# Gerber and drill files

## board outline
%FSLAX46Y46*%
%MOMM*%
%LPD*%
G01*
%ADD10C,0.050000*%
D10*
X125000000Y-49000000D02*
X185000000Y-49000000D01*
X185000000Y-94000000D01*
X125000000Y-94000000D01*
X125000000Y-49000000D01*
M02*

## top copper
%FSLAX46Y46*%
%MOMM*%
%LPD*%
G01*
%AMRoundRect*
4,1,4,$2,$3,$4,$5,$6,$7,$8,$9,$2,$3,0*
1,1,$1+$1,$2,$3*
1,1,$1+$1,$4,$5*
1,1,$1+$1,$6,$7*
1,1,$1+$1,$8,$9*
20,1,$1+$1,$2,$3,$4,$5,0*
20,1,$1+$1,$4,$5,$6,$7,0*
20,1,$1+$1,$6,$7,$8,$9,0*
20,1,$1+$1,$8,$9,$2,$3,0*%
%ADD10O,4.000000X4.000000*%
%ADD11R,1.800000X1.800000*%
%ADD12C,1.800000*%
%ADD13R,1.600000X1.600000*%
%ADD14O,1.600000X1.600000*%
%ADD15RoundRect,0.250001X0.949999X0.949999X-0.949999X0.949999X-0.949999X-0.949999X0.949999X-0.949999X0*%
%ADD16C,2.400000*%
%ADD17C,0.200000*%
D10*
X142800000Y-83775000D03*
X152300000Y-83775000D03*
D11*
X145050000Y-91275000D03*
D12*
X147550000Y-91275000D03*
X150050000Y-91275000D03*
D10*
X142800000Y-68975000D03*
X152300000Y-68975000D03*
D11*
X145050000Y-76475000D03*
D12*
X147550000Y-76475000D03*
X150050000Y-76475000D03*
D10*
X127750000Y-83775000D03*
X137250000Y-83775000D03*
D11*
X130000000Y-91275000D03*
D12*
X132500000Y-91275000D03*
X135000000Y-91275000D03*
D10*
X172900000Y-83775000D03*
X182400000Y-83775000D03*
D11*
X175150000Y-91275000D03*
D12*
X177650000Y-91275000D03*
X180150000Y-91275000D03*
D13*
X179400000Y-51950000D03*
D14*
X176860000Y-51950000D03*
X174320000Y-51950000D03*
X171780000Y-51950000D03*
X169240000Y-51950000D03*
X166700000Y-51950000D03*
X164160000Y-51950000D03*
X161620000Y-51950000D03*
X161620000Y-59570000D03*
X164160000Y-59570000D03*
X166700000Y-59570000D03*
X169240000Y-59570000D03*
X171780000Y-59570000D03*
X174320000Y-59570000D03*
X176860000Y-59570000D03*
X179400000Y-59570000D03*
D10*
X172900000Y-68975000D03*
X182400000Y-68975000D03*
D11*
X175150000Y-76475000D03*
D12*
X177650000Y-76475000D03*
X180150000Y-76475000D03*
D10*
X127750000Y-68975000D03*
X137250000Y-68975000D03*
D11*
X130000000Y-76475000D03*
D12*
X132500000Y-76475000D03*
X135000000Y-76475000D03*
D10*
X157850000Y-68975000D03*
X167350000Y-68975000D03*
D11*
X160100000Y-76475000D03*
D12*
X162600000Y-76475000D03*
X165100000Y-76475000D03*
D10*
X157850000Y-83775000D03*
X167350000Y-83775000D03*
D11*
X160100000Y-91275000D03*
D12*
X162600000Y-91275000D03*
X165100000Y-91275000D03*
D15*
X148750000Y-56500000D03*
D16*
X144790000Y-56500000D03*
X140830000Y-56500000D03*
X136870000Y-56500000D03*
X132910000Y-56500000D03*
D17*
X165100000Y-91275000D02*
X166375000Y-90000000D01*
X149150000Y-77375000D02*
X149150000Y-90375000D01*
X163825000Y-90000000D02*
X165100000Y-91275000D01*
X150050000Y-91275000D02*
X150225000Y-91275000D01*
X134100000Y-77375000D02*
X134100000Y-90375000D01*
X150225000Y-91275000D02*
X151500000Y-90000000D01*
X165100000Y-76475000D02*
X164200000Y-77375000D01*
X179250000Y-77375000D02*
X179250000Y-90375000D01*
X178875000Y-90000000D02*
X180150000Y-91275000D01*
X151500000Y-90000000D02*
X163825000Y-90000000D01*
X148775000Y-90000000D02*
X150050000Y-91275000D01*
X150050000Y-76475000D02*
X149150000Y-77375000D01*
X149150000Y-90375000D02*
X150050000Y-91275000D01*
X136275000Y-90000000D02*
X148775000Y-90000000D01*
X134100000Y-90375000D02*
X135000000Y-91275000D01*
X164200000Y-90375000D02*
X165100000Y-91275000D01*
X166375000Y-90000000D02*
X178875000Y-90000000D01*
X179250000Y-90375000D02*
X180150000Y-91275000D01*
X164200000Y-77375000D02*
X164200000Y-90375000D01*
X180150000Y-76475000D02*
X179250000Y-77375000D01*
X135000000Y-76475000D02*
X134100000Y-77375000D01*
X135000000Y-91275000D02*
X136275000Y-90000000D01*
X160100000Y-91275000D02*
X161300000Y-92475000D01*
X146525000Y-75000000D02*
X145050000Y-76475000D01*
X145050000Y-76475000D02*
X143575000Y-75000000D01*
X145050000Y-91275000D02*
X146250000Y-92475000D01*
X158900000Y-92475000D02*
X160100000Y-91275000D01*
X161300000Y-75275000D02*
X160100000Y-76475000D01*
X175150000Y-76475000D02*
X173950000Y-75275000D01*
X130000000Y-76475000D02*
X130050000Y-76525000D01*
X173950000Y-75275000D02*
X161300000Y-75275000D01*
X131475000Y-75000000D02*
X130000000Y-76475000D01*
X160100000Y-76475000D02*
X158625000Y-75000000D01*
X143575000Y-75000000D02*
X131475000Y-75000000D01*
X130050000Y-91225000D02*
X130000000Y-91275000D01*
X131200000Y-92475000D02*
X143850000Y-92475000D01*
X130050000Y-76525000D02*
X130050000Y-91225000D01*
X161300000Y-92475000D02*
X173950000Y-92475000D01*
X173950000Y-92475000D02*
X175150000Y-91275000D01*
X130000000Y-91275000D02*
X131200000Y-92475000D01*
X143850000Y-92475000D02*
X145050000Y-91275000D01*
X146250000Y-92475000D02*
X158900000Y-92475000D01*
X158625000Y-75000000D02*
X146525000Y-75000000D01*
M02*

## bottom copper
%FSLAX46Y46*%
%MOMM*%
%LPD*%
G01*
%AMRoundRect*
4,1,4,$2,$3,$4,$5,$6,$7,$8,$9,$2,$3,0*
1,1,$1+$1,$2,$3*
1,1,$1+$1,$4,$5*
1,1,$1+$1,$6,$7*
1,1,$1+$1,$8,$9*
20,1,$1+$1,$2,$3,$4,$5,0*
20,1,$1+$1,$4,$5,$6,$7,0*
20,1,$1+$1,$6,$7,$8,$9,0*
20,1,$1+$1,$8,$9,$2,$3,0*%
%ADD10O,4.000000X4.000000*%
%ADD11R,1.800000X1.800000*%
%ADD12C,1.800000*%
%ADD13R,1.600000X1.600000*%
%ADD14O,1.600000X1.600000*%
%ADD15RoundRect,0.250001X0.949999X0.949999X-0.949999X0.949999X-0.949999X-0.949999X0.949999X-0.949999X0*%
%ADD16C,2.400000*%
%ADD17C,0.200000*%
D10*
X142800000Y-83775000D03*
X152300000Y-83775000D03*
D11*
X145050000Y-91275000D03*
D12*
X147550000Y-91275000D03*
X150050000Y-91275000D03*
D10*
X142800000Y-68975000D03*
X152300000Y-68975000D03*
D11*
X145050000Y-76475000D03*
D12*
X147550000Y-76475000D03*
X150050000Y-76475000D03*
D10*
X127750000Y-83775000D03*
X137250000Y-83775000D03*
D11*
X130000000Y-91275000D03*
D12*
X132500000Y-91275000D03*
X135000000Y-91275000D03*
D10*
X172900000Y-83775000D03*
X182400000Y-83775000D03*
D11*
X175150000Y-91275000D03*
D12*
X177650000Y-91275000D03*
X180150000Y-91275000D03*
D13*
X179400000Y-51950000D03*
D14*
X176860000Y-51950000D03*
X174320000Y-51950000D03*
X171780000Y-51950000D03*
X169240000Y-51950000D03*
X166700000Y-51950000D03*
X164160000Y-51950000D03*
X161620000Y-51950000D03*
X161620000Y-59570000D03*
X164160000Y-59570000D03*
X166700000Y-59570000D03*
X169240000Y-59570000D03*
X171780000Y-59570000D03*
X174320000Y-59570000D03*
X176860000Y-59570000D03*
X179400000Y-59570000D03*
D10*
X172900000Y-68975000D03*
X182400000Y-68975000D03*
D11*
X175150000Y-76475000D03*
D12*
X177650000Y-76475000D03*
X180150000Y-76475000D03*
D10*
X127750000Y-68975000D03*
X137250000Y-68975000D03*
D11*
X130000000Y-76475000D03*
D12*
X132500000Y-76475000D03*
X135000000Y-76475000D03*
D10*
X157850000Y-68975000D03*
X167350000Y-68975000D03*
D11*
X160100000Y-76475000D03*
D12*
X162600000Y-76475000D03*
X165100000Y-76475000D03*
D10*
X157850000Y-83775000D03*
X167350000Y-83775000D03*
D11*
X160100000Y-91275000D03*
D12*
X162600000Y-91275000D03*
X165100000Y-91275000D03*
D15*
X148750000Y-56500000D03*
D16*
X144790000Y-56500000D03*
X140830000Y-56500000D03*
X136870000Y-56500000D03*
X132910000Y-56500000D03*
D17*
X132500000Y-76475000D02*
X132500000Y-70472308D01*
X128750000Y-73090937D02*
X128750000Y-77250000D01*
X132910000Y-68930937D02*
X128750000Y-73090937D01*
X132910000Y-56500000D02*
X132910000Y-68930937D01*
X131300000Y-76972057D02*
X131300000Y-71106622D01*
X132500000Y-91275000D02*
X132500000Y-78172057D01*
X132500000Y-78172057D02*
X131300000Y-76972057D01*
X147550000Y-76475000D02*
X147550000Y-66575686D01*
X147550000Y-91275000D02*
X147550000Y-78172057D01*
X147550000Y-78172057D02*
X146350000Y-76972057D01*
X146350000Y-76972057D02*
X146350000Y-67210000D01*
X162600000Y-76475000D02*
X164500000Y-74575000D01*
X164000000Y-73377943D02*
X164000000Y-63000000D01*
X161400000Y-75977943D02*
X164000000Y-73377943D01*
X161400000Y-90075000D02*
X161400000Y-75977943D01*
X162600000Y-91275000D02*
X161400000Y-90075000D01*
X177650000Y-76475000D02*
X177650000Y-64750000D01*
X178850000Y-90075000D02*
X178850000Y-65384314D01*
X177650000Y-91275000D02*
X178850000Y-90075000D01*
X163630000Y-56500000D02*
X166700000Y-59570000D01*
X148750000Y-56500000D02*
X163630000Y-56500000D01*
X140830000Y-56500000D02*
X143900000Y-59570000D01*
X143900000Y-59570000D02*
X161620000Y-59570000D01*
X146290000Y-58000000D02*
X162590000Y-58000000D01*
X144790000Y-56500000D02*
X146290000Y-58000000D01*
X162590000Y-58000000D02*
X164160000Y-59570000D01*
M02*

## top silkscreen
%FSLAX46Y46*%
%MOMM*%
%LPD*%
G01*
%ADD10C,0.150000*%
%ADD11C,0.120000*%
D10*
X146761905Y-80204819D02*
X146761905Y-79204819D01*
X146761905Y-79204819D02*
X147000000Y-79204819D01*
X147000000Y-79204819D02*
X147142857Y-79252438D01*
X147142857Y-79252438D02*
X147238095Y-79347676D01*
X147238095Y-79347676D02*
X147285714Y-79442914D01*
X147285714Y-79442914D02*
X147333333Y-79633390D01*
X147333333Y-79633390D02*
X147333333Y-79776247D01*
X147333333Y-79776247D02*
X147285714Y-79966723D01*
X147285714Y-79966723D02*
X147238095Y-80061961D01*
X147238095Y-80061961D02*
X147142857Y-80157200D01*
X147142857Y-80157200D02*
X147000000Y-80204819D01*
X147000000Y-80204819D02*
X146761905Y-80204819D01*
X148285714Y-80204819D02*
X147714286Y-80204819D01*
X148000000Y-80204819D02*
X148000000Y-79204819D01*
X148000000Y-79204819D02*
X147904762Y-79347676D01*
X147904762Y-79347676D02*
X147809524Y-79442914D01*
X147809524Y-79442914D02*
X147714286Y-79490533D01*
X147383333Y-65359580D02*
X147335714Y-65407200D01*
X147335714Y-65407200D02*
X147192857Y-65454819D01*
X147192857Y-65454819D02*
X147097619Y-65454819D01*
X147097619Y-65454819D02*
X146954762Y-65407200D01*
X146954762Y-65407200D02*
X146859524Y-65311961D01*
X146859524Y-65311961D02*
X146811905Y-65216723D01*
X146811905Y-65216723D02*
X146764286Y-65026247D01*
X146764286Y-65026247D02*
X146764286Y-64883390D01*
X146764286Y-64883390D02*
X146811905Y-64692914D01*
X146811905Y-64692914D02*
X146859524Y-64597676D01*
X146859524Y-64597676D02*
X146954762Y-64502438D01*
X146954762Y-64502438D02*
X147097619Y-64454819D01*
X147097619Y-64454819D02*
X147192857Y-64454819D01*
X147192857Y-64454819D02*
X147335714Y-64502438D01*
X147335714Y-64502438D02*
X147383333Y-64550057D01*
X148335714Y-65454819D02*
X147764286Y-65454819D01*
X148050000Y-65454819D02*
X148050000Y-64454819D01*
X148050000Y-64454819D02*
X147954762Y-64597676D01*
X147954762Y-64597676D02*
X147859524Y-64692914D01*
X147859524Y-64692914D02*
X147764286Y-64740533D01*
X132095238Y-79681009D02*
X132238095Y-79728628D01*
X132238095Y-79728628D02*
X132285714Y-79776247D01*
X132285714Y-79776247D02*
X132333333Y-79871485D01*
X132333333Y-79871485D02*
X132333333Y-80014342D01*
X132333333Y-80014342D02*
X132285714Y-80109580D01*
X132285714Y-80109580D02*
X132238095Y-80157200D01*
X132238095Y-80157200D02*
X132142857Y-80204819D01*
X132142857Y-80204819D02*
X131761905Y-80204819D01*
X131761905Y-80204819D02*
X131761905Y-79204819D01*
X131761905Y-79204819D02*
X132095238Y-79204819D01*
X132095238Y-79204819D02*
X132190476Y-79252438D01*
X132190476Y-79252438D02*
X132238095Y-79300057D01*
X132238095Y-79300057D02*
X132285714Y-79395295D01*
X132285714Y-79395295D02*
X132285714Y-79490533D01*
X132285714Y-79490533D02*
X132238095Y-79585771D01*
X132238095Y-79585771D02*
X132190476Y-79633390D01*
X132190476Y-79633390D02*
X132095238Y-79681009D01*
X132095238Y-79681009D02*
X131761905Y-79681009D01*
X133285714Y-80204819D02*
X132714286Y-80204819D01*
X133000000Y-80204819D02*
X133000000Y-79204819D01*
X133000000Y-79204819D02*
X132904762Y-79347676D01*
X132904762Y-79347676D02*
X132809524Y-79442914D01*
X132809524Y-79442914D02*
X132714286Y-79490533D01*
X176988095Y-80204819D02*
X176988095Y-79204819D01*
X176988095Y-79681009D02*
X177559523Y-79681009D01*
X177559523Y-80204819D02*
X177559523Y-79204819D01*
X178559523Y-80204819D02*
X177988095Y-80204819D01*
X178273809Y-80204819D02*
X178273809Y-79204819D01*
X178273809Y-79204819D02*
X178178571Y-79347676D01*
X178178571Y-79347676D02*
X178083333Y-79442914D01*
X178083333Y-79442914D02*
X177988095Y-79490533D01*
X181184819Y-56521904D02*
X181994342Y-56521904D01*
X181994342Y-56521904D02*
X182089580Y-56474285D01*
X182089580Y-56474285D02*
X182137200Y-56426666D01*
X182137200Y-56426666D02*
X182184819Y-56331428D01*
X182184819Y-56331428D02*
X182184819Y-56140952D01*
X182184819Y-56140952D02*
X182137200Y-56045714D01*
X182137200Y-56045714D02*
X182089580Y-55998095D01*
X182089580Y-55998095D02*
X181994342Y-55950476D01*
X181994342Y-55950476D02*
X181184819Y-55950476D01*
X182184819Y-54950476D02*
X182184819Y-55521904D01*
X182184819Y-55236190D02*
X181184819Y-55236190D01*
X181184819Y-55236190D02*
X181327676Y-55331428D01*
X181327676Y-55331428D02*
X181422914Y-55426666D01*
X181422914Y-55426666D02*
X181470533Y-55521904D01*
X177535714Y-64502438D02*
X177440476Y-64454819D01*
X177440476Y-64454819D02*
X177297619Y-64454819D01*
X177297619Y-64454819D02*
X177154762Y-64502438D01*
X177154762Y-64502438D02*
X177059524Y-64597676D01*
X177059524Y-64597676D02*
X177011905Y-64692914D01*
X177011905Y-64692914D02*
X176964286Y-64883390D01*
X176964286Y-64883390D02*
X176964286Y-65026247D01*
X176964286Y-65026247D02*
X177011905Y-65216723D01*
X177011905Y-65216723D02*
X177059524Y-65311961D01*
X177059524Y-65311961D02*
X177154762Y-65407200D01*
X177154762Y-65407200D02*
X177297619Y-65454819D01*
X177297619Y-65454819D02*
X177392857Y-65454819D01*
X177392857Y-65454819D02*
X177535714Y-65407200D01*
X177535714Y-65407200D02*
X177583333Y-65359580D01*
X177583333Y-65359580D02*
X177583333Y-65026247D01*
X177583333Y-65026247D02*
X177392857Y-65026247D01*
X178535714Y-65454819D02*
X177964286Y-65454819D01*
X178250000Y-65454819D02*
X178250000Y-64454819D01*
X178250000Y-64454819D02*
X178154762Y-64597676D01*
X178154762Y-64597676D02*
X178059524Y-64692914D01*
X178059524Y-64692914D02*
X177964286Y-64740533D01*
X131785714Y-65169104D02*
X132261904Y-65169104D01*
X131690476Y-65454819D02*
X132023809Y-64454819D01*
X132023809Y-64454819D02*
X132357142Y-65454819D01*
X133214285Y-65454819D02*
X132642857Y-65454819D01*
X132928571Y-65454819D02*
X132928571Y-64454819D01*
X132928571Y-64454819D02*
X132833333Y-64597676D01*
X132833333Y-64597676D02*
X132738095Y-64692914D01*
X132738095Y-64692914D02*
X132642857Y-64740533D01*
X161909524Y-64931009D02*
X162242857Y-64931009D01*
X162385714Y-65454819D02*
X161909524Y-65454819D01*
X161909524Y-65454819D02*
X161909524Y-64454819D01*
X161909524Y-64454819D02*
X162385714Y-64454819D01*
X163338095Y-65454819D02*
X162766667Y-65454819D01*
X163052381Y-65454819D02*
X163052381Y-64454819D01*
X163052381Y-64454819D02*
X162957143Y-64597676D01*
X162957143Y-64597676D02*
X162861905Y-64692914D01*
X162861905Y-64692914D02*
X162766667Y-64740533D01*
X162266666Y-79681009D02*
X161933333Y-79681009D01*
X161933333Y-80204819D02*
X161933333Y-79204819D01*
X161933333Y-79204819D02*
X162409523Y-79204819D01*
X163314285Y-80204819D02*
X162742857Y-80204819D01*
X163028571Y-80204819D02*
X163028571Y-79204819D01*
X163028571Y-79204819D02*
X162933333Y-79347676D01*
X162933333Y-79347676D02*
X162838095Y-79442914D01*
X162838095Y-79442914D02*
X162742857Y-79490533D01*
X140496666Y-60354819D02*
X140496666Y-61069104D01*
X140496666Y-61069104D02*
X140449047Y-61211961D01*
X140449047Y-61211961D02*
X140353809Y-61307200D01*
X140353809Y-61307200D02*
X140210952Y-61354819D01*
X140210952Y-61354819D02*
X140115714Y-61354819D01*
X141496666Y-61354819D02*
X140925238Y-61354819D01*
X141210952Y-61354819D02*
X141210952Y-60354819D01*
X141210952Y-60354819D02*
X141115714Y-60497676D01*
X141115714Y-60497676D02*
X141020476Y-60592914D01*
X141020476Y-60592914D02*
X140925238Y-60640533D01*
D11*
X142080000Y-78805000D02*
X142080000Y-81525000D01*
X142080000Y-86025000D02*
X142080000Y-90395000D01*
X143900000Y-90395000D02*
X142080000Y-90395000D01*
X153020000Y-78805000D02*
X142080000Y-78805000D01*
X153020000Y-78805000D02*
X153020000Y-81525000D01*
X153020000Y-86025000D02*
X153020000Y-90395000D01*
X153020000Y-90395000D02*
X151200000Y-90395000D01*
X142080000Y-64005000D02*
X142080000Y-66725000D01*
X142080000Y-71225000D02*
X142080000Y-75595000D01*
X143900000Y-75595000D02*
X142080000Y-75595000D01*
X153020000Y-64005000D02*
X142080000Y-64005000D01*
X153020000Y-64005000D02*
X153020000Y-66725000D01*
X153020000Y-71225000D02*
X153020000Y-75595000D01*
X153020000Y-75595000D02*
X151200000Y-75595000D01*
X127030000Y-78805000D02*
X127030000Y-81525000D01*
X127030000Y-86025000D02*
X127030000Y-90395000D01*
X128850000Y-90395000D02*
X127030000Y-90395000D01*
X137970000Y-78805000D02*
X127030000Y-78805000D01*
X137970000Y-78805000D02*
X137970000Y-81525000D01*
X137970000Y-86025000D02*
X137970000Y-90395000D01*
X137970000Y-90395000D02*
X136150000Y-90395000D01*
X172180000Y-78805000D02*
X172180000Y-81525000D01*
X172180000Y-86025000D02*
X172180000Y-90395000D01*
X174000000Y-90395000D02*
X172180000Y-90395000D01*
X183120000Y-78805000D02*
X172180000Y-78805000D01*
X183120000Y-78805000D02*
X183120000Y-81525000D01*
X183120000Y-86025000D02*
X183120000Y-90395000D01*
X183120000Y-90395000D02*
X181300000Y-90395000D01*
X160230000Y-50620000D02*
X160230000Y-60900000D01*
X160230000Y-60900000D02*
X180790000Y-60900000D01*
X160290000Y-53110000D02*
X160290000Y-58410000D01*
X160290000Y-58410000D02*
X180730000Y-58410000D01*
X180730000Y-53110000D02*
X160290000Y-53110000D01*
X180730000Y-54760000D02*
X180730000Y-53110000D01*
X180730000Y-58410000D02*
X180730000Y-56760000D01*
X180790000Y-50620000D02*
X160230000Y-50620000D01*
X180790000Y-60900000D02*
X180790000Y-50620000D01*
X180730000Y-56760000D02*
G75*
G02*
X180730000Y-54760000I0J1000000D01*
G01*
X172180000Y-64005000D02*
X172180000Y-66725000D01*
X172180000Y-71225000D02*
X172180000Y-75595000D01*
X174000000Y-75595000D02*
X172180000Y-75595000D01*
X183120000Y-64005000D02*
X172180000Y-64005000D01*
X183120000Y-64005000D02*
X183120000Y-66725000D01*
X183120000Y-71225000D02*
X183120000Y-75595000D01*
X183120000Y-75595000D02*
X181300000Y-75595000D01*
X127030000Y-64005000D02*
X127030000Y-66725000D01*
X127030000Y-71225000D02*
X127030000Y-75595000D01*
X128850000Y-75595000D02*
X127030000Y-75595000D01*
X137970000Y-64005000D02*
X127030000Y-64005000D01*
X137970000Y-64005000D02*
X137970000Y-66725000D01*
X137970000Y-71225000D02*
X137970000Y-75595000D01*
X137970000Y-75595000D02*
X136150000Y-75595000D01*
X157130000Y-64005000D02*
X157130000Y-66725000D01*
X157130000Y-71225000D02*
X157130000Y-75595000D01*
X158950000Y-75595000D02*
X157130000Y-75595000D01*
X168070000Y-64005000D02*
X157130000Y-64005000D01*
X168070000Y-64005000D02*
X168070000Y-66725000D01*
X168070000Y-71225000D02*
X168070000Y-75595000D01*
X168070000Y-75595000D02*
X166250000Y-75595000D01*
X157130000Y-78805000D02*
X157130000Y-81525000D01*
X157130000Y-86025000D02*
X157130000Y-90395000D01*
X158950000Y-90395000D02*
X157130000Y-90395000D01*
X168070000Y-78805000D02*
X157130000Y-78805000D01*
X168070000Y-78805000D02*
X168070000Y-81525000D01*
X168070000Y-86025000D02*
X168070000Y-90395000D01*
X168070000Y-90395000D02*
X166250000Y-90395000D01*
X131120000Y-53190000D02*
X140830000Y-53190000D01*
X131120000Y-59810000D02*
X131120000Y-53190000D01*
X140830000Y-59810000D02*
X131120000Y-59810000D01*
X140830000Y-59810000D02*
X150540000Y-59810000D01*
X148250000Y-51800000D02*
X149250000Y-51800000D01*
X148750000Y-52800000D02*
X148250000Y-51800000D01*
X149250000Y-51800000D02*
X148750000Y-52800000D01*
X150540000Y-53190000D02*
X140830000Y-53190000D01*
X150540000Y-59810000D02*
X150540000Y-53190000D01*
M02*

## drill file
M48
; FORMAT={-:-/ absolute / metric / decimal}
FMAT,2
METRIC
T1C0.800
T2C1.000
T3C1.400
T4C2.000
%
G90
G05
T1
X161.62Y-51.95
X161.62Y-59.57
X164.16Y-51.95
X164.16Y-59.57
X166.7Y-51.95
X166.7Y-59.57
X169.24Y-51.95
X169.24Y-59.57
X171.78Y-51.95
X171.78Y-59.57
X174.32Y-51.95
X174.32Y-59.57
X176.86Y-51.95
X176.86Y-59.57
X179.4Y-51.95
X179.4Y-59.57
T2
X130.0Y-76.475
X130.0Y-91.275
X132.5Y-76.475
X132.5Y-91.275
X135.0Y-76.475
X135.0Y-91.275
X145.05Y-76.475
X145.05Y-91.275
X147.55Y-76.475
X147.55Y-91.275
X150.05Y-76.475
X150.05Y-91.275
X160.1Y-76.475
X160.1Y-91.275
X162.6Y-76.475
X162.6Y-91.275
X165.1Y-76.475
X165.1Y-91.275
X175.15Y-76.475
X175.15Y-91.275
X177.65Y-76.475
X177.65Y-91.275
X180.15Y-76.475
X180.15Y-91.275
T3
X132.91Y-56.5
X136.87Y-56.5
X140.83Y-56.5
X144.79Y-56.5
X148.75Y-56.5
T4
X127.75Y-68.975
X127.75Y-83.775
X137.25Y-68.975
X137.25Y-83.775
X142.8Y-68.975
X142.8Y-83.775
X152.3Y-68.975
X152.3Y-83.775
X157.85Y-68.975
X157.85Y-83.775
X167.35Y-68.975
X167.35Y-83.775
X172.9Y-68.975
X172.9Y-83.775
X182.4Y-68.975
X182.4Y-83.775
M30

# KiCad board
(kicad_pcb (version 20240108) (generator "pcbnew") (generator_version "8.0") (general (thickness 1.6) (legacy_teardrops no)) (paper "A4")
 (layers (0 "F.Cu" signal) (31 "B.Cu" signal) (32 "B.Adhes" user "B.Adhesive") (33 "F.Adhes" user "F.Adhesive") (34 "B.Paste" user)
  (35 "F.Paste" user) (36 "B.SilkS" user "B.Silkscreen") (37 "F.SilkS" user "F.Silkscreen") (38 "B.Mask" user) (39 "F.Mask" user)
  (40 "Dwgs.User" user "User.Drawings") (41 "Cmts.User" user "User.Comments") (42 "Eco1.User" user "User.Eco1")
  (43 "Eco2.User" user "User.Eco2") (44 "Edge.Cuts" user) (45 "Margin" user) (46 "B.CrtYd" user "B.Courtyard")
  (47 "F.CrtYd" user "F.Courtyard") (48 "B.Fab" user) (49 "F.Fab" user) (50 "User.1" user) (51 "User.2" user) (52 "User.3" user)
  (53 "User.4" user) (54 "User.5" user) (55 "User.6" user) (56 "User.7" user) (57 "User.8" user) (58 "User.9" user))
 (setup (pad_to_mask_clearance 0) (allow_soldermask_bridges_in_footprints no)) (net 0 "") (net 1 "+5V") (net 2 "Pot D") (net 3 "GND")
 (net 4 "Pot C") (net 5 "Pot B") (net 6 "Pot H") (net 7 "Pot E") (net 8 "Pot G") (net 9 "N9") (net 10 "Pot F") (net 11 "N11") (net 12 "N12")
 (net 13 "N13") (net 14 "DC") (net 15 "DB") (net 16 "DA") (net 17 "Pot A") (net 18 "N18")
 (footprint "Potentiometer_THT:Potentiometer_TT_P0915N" (layer "F.Cu") (at 145.05 91.275)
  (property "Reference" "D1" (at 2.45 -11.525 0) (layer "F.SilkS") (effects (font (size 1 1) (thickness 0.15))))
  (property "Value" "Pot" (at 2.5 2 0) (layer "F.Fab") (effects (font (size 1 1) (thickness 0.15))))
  (fp_line (start -2.97 -12.47) (end -2.97 -9.75) (stroke (width 0.12) (type solid)) (layer "F.SilkS"))
  (fp_line (start -2.97 -5.25) (end -2.97 -0.88) (stroke (width 0.12) (type solid)) (layer "F.SilkS"))
  (fp_line (start -1.15 -0.88) (end -2.97 -0.88) (stroke (width 0.12) (type solid)) (layer "F.SilkS"))
  (fp_line (start 7.97 -12.47) (end -2.97 -12.47) (stroke (width 0.12) (type solid)) (layer "F.SilkS"))
  (fp_line (start 7.97 -12.47) (end 7.97 -9.75) (stroke (width 0.12) (type solid)) (layer "F.SilkS"))
  (fp_line (start 7.97 -5.25) (end 7.97 -0.88) (stroke (width 0.12) (type solid)) (layer "F.SilkS"))
  (fp_line (start 7.97 -0.88) (end 6.15 -0.88) (stroke (width 0.12) (type solid)) (layer "F.SilkS"))
  (pad "" thru_hole oval (at -2.25 -7.5) (size 4 4) (drill 2) (layers "*.Cu" "*.Mask") (remove_unused_layers no))
  (pad "" thru_hole oval (at 7.25 -7.5) (size 4 4) (drill 2) (layers "*.Cu" "*.Mask") (remove_unused_layers no))
  (pad "1" thru_hole rect (at 0 0) (size 1.8 1.8) (drill 1) (layers "*.Cu" "*.Mask") (remove_unused_layers no) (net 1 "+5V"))
  (pad "2" thru_hole circle (at 2.5 0) (size 1.8 1.8) (drill 1) (layers "*.Cu" "*.Mask") (remove_unused_layers no) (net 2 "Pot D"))
  (pad "3" thru_hole circle (at 5 0) (size 1.8 1.8) (drill 1) (layers "*.Cu" "*.Mask") (remove_unused_layers no) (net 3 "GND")))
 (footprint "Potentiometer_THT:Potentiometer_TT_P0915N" (layer "F.Cu") (at 145.05 76.475)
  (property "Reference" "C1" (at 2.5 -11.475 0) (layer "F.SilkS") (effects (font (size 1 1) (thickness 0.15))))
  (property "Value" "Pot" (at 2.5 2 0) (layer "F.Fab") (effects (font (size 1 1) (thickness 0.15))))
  (fp_line (start -2.97 -12.47) (end -2.97 -9.75) (stroke (width 0.12) (type solid)) (layer "F.SilkS"))
  (fp_line (start -2.97 -5.25) (end -2.97 -0.88) (stroke (width 0.12) (type solid)) (layer "F.SilkS"))
  (fp_line (start -1.15 -0.88) (end -2.97 -0.88) (stroke (width 0.12) (type solid)) (layer "F.SilkS"))
  (fp_line (start 7.97 -12.47) (end -2.97 -12.47) (stroke (width 0.12) (type solid)) (layer "F.SilkS"))
  (fp_line (start 7.97 -12.47) (end 7.97 -9.75) (stroke (width 0.12) (type solid)) (layer "F.SilkS"))
  (fp_line (start 7.97 -5.25) (end 7.97 -0.88) (stroke (width 0.12) (type solid)) (layer "F.SilkS"))
  (fp_line (start 7.97 -0.88) (end 6.15 -0.88) (stroke (width 0.12) (type solid)) (layer "F.SilkS"))
  (pad "" thru_hole oval (at -2.25 -7.5) (size 4 4) (drill 2) (layers "*.Cu" "*.Mask") (remove_unused_layers no))
  (pad "" thru_hole oval (at 7.25 -7.5) (size 4 4) (drill 2) (layers "*.Cu" "*.Mask") (remove_unused_layers no))
  (pad "1" thru_hole rect (at 0 0) (size 1.8 1.8) (drill 1) (layers "*.Cu" "*.Mask") (remove_unused_layers no) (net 1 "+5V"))
  (pad "2" thru_hole circle (at 2.5 0) (size 1.8 1.8) (drill 1) (layers "*.Cu" "*.Mask") (remove_unused_layers no) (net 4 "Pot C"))
  (pad "3" thru_hole circle (at 5 0) (size 1.8 1.8) (drill 1) (layers "*.Cu" "*.Mask") (remove_unused_layers no) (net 3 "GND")))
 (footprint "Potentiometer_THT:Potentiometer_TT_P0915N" (layer "F.Cu") (at 130 91.275)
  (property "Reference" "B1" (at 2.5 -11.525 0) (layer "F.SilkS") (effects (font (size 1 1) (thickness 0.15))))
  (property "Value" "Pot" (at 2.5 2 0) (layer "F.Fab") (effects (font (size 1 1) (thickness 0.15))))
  (fp_line (start -2.97 -12.47) (end -2.97 -9.75) (stroke (width 0.12) (type solid)) (layer "F.SilkS"))
  (fp_line (start -2.97 -5.25) (end -2.97 -0.88) (stroke (width 0.12) (type solid)) (layer "F.SilkS"))
  (fp_line (start -1.15 -0.88) (end -2.97 -0.88) (stroke (width 0.12) (type solid)) (layer "F.SilkS"))
  (fp_line (start 7.97 -12.47) (end -2.97 -12.47) (stroke (width 0.12) (type solid)) (layer "F.SilkS"))
  (fp_line (start 7.97 -12.47) (end 7.97 -9.75) (stroke (width 0.12) (type solid)) (layer "F.SilkS"))
  (fp_line (start 7.97 -5.25) (end 7.97 -0.88) (stroke (width 0.12) (type solid)) (layer "F.SilkS"))
  (fp_line (start 7.97 -0.88) (end 6.15 -0.88) (stroke (width 0.12) (type solid)) (layer "F.SilkS"))
  (pad "" thru_hole oval (at -2.25 -7.5) (size 4 4) (drill 2) (layers "*.Cu" "*.Mask") (remove_unused_layers no))
  (pad "" thru_hole oval (at 7.25 -7.5) (size 4 4) (drill 2) (layers "*.Cu" "*.Mask") (remove_unused_layers no))
  (pad "1" thru_hole rect (at 0 0) (size 1.8 1.8) (drill 1) (layers "*.Cu" "*.Mask") (remove_unused_layers no) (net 1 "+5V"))
  (pad "2" thru_hole circle (at 2.5 0) (size 1.8 1.8) (drill 1) (layers "*.Cu" "*.Mask") (remove_unused_layers no) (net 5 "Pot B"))
  (pad "3" thru_hole circle (at 5 0) (size 1.8 1.8) (drill 1) (layers "*.Cu" "*.Mask") (remove_unused_layers no) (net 3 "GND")))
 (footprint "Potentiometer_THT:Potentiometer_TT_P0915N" (layer "F.Cu") (at 175.15 91.275)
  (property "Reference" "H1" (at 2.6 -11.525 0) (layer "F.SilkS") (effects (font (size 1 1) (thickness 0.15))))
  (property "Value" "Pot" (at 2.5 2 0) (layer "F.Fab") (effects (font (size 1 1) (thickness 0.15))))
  (fp_line (start -2.97 -12.47) (end -2.97 -9.75) (stroke (width 0.12) (type solid)) (layer "F.SilkS"))
  (fp_line (start -2.97 -5.25) (end -2.97 -0.88) (stroke (width 0.12) (type solid)) (layer "F.SilkS"))
  (fp_line (start -1.15 -0.88) (end -2.97 -0.88) (stroke (width 0.12) (type solid)) (layer "F.SilkS"))
  (fp_line (start 7.97 -12.47) (end -2.97 -12.47) (stroke (width 0.12) (type solid)) (layer "F.SilkS"))
  (fp_line (start 7.97 -12.47) (end 7.97 -9.75) (stroke (width 0.12) (type solid)) (layer "F.SilkS"))
  (fp_line (start 7.97 -5.25) (end 7.97 -0.88) (stroke (width 0.12) (type solid)) (layer "F.SilkS"))
  (fp_line (start 7.97 -0.88) (end 6.15 -0.88) (stroke (width 0.12) (type solid)) (layer "F.SilkS"))
  (pad "" thru_hole oval (at -2.25 -7.5) (size 4 4) (drill 2) (layers "*.Cu" "*.Mask") (remove_unused_layers no))
  (pad "" thru_hole oval (at 7.25 -7.5) (size 4 4) (drill 2) (layers "*.Cu" "*.Mask") (remove_unused_layers no))
  (pad "1" thru_hole rect (at 0 0) (size 1.8 1.8) (drill 1) (layers "*.Cu" "*.Mask") (remove_unused_layers no) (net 1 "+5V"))
  (pad "2" thru_hole circle (at 2.5 0) (size 1.8 1.8) (drill 1) (layers "*.Cu" "*.Mask") (remove_unused_layers no) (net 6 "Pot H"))
  (pad "3" thru_hole circle (at 5 0) (size 1.8 1.8) (drill 1) (layers "*.Cu" "*.Mask") (remove_unused_layers no) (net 3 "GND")))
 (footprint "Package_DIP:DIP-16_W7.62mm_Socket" (layer "F.Cu") (at 179.4 51.95 -90)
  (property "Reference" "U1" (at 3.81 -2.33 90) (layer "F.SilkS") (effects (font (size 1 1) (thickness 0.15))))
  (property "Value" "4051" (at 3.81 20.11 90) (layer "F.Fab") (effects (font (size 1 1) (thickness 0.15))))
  (fp_line (start -1.33 19.17) (end 8.95 19.17) (stroke (width 0.12) (type solid)) (layer "F.SilkS"))
  (fp_line (start 8.95 19.17) (end 8.95 -1.39) (stroke (width 0.12) (type solid)) (layer "F.SilkS"))
  (fp_line (start 1.16 19.11) (end 6.46 19.11) (stroke (width 0.12) (type solid)) (layer "F.SilkS"))
  (fp_line (start 6.46 19.11) (end 6.46 -1.33) (stroke (width 0.12) (type solid)) (layer "F.SilkS"))
  (fp_line (start 1.16 -1.33) (end 1.16 19.11) (stroke (width 0.12) (type solid)) (layer "F.SilkS"))
  (fp_line (start 2.81 -1.33) (end 1.16 -1.33) (stroke (width 0.12) (type solid)) (layer "F.SilkS"))
  (fp_line (start 6.46 -1.33) (end 4.81 -1.33) (stroke (width 0.12) (type solid)) (layer "F.SilkS"))
  (fp_line (start -1.33 -1.39) (end -1.33 19.17) (stroke (width 0.12) (type solid)) (layer "F.SilkS"))
  (fp_line (start 8.95 -1.39) (end -1.33 -1.39) (stroke (width 0.12) (type solid)) (layer "F.SilkS"))
  (fp_arc (start 4.81 -1.33) (mid 3.81 -0.33) (end 2.81 -1.33) (stroke (width 0.12) (type solid)) (layer "F.SilkS"))
  (pad "1" thru_hole rect (at 0 0 270) (size 1.6 1.6) (drill 0.8) (layers "*.Cu" "*.Mask") (remove_unused_layers no) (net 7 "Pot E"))
  (pad "2" thru_hole oval (at 0 2.54 270) (size 1.6 1.6) (drill 0.8) (layers "*.Cu" "*.Mask") (remove_unused_layers no) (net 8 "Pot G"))
  (pad "3" thru_hole oval (at 0 5.08 270) (size 1.6 1.6) (drill 0.8) (layers "*.Cu" "*.Mask") (remove_unused_layers no) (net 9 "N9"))
  (pad "4" thru_hole oval (at 0 7.62 270) (size 1.6 1.6) (drill 0.8) (layers "*.Cu" "*.Mask") (remove_unused_layers no) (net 6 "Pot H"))
  (pad "5" thru_hole oval (at 0 10.16 270) (size 1.6 1.6) (drill 0.8) (layers "*.Cu" "*.Mask") (remove_unused_layers no) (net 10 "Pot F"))
  (pad "6" thru_hole oval (at 0 12.7 270) (size 1.6 1.6) (drill 0.8) (layers "*.Cu" "*.Mask") (remove_unused_layers no) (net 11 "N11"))
  (pad "7" thru_hole oval (at 0 15.24 270) (size 1.6 1.6) (drill 0.8) (layers "*.Cu" "*.Mask") (remove_unused_layers no) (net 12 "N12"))
  (pad "8" thru_hole oval (at 0 17.78 270) (size 1.6 1.6) (drill 0.8) (layers "*.Cu" "*.Mask") (remove_unused_layers no) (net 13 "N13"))
  (pad "9" thru_hole oval (at 7.62 17.78 270) (size 1.6 1.6) (drill 0.8) (layers "*.Cu" "*.Mask") (remove_unused_layers no) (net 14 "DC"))
  (pad "10" thru_hole oval (at 7.62 15.24 270) (size 1.6 1.6) (drill 0.8) (layers "*.Cu" "*.Mask") (remove_unused_layers no) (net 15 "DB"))
  (pad "11" thru_hole oval (at 7.62 12.7 270) (size 1.6 1.6) (drill 0.8) (layers "*.Cu" "*.Mask") (remove_unused_layers no) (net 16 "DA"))
  (pad "12" thru_hole oval (at 7.62 10.16 270) (size 1.6 1.6) (drill 0.8) (layers "*.Cu" "*.Mask") (remove_unused_layers no) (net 2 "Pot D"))
  (pad "13" thru_hole oval (at 7.62 7.62 270) (size 1.6 1.6) (drill 0.8) (layers "*.Cu" "*.Mask") (remove_unused_layers no) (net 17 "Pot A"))
  (pad "14" thru_hole oval (at 7.62 5.08 270) (size 1.6 1.6) (drill 0.8) (layers "*.Cu" "*.Mask") (remove_unused_layers no) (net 5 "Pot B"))
  (pad "15" thru_hole oval (at 7.62 2.54 270) (size 1.6 1.6) (drill 0.8) (layers "*.Cu" "*.Mask") (remove_unused_layers no) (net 4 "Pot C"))
  (pad "16" thru_hole oval (at 7.62 0 270) (size 1.6 1.6) (drill 0.8) (layers "*.Cu" "*.Mask") (remove_unused_layers no) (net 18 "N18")))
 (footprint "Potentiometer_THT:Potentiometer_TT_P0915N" (layer "F.Cu") (at 175.15 76.475)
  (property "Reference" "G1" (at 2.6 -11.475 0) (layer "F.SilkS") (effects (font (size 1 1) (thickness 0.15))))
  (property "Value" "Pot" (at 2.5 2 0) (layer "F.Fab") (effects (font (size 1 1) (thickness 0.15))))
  (fp_line (start -2.97 -12.47) (end -2.97 -9.75) (stroke (width 0.12) (type solid)) (layer "F.SilkS"))
  (fp_line (start -2.97 -5.25) (end -2.97 -0.88) (stroke (width 0.12) (type solid)) (layer "F.SilkS"))
  (fp_line (start -1.15 -0.88) (end -2.97 -0.88) (stroke (width 0.12) (type solid)) (layer "F.SilkS"))
  (fp_line (start 7.97 -12.47) (end -2.97 -12.47) (stroke (width 0.12) (type solid)) (layer "F.SilkS"))
  (fp_line (start 7.97 -12.47) (end 7.97 -9.75) (stroke (width 0.12) (type solid)) (layer "F.SilkS"))
  (fp_line (start 7.97 -5.25) (end 7.97 -0.88) (stroke (width 0.12) (type solid)) (layer "F.SilkS"))
  (fp_line (start 7.97 -0.88) (end 6.15 -0.88) (stroke (width 0.12) (type solid)) (layer "F.SilkS"))
  (pad "" thru_hole oval (at -2.25 -7.5) (size 4 4) (drill 2) (layers "*.Cu" "*.Mask") (remove_unused_layers no))
  (pad "" thru_hole oval (at 7.25 -7.5) (size 4 4) (drill 2) (layers "*.Cu" "*.Mask") (remove_unused_layers no))
  (pad "1" thru_hole rect (at 0 0) (size 1.8 1.8) (drill 1) (layers "*.Cu" "*.Mask") (remove_unused_layers no) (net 1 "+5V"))
  (pad "2" thru_hole circle (at 2.5 0) (size 1.8 1.8) (drill 1) (layers "*.Cu" "*.Mask") (remove_unused_layers no) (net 8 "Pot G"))
  (pad "3" thru_hole circle (at 5 0) (size 1.8 1.8) (drill 1) (layers "*.Cu" "*.Mask") (remove_unused_layers no) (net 3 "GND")))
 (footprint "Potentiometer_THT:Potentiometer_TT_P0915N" (layer "F.Cu") (at 130 76.475)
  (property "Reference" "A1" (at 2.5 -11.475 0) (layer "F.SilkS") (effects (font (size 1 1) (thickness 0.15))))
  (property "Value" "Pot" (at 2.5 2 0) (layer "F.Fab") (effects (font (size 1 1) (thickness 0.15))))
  (fp_line (start -2.97 -12.47) (end -2.97 -9.75) (stroke (width 0.12) (type solid)) (layer "F.SilkS"))
  (fp_line (start -2.97 -5.25) (end -2.97 -0.88) (stroke (width 0.12) (type solid)) (layer "F.SilkS"))
  (fp_line (start -1.15 -0.88) (end -2.97 -0.88) (stroke (width 0.12) (type solid)) (layer "F.SilkS"))
  (fp_line (start 7.97 -12.47) (end -2.97 -12.47) (stroke (width 0.12) (type solid)) (layer "F.SilkS"))
  (fp_line (start 7.97 -12.47) (end 7.97 -9.75) (stroke (width 0.12) (type solid)) (layer "F.SilkS"))
  (fp_line (start 7.97 -5.25) (end 7.97 -0.88) (stroke (width 0.12) (type solid)) (layer "F.SilkS"))
  (fp_line (start 7.97 -0.88) (end 6.15 -0.88) (stroke (width 0.12) (type solid)) (layer "F.SilkS"))
  (pad "" thru_hole oval (at -2.25 -7.5) (size 4 4) (drill 2) (layers "*.Cu" "*.Mask") (remove_unused_layers no))
  (pad "" thru_hole oval (at 7.25 -7.5) (size 4 4) (drill 2) (layers "*.Cu" "*.Mask") (remove_unused_layers no))
  (pad "1" thru_hole rect (at 0 0) (size 1.8 1.8) (drill 1) (layers "*.Cu" "*.Mask") (remove_unused_layers no) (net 1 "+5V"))
  (pad "2" thru_hole circle (at 2.5 0) (size 1.8 1.8) (drill 1) (layers "*.Cu" "*.Mask") (remove_unused_layers no) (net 17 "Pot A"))
  (pad "3" thru_hole circle (at 5 0) (size 1.8 1.8) (drill 1) (layers "*.Cu" "*.Mask") (remove_unused_layers no) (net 3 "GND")))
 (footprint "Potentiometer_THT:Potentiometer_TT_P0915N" (layer "F.Cu") (at 160.1 76.475)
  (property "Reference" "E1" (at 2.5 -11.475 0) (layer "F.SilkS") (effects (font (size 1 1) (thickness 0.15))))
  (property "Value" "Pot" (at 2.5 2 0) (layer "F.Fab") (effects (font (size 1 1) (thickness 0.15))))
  (fp_line (start -2.97 -12.47) (end -2.97 -9.75) (stroke (width 0.12) (type solid)) (layer "F.SilkS"))
  (fp_line (start -2.97 -5.25) (end -2.97 -0.88) (stroke (width 0.12) (type solid)) (layer "F.SilkS"))
  (fp_line (start -1.15 -0.88) (end -2.97 -0.88) (stroke (width 0.12) (type solid)) (layer "F.SilkS"))
  (fp_line (start 7.97 -12.47) (end -2.97 -12.47) (stroke (width 0.12) (type solid)) (layer "F.SilkS"))
  (fp_line (start 7.97 -12.47) (end 7.97 -9.75) (stroke (width 0.12) (type solid)) (layer "F.SilkS"))
  (fp_line (start 7.97 -5.25) (end 7.97 -0.88) (stroke (width 0.12) (type solid)) (layer "F.SilkS"))
  (fp_line (start 7.97 -0.88) (end 6.15 -0.88) (stroke (width 0.12) (type solid)) (layer "F.SilkS"))
  (pad "" thru_hole oval (at -2.25 -7.5) (size 4 4) (drill 2) (layers "*.Cu" "*.Mask") (remove_unused_layers no))
  (pad "" thru_hole oval (at 7.25 -7.5) (size 4 4) (drill 2) (layers "*.Cu" "*.Mask") (remove_unused_layers no))
  (pad "1" thru_hole rect (at 0 0) (size 1.8 1.8) (drill 1) (layers "*.Cu" "*.Mask") (remove_unused_layers no) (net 1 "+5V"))
  (pad "2" thru_hole circle (at 2.5 0) (size 1.8 1.8) (drill 1) (layers "*.Cu" "*.Mask") (remove_unused_layers no) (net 7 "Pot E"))
  (pad "3" thru_hole circle (at 5 0) (size 1.8 1.8) (drill 1) (layers "*.Cu" "*.Mask") (remove_unused_layers no) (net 3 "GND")))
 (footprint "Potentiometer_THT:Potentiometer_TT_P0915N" (layer "F.Cu") (at 160.1 91.275)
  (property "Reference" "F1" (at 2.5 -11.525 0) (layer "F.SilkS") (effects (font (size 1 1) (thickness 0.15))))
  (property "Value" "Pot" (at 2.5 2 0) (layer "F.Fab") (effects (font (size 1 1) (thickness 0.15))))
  (fp_line (start -2.97 -12.47) (end -2.97 -9.75) (stroke (width 0.12) (type solid)) (layer "F.SilkS"))
  (fp_line (start -2.97 -5.25) (end -2.97 -0.88) (stroke (width 0.12) (type solid)) (layer "F.SilkS"))
  (fp_line (start -1.15 -0.88) (end -2.97 -0.88) (stroke (width 0.12) (type solid)) (layer "F.SilkS"))
  (fp_line (start 7.97 -12.47) (end -2.97 -12.47) (stroke (width 0.12) (type solid)) (layer "F.SilkS"))
  (fp_line (start 7.97 -12.47) (end 7.97 -9.75) (stroke (width 0.12) (type solid)) (layer "F.SilkS"))
  (fp_line (start 7.97 -5.25) (end 7.97 -0.88) (stroke (width 0.12) (type solid)) (layer "F.SilkS"))
  (fp_line (start 7.97 -0.88) (end 6.15 -0.88) (stroke (width 0.12) (type solid)) (layer "F.SilkS"))
  (pad "" thru_hole oval (at -2.25 -7.5) (size 4 4) (drill 2) (layers "*.Cu" "*.Mask") (remove_unused_layers no))
  (pad "" thru_hole oval (at 7.25 -7.5) (size 4 4) (drill 2) (layers "*.Cu" "*.Mask") (remove_unused_layers no))
  (pad "1" thru_hole rect (at 0 0) (size 1.8 1.8) (drill 1) (layers "*.Cu" "*.Mask") (remove_unused_layers no) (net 1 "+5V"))
  (pad "2" thru_hole circle (at 2.5 0) (size 1.8 1.8) (drill 1) (layers "*.Cu" "*.Mask") (remove_unused_layers no) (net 10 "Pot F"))
  (pad "3" thru_hole circle (at 5 0) (size 1.8 1.8) (drill 1) (layers "*.Cu" "*.Mask") (remove_unused_layers no) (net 3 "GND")))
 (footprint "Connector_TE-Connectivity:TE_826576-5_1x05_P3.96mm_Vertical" (layer "F.Cu") (at 148.75 56.5 180)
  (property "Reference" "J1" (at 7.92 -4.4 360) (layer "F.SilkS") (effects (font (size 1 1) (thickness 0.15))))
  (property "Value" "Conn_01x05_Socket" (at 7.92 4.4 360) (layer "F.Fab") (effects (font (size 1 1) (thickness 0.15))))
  (fp_line (start 17.63 3.31) (end 7.92 3.31) (stroke (width 0.12) (type solid)) (layer "F.SilkS"))
  (fp_line (start 17.63 -3.31) (end 17.63 3.31) (stroke (width 0.12) (type solid)) (layer "F.SilkS"))
  (fp_line (start 7.92 -3.31) (end 17.63 -3.31) (stroke (width 0.12) (type solid)) (layer "F.SilkS"))
  (fp_line (start 7.92 -3.31) (end -1.79 -3.31) (stroke (width 0.12) (type solid)) (layer "F.SilkS"))
  (fp_line (start 0.5 4.7) (end -0.5 4.7) (stroke (width 0.12) (type solid)) (layer "F.SilkS"))
  (fp_line (start 0 3.7) (end 0.5 4.7) (stroke (width 0.12) (type solid)) (layer "F.SilkS"))
  (fp_line (start -0.5 4.7) (end 0 3.7) (stroke (width 0.12) (type solid)) (layer "F.SilkS"))
  (fp_line (start -1.79 3.31) (end 7.92 3.31) (stroke (width 0.12) (type solid)) (layer "F.SilkS"))
  (fp_line (start -1.79 -3.31) (end -1.79 3.31) (stroke (width 0.12) (type solid)) (layer "F.SilkS"))
  (pad "1" thru_hole roundrect (at 0 0 180) (size 2.4 2.4) (drill 1.4) (layers "*.Cu" "*.Mask") (remove_unused_layers no)
   (roundrect_rratio 0.104167) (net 16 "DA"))
  (pad "2" thru_hole circle (at 3.96 0 180) (size 2.4 2.4) (drill 1.4) (layers "*.Cu" "*.Mask") (remove_unused_layers no) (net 15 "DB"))
  (pad "3" thru_hole circle (at 7.92 0 180) (size 2.4 2.4) (drill 1.4) (layers "*.Cu" "*.Mask") (remove_unused_layers no) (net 14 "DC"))
  (pad "4" thru_hole circle (at 11.88 0 180) (size 2.4 2.4) (drill 1.4) (layers "*.Cu" "*.Mask") (remove_unused_layers no) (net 1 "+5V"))
  (pad "5" thru_hole circle (at 15.84 0 180) (size 2.4 2.4) (drill 1.4) (layers "*.Cu" "*.Mask") (remove_unused_layers no) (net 3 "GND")))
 (gr_rect (start 125 49) (end 185 94) (stroke (width 0.05) (type default)) (fill none) (layer "Edge.Cuts"))
 (segment (start 132.5 76.475) (end 132.5 70.472308) (width 0.2) (layer "B.Cu") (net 17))
 (segment (start 165.1 91.275) (end 166.375 90) (width 0.2) (layer "F.Cu") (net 3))
 (segment (start 149.15 77.375) (end 149.15 90.375) (width 0.2) (layer "F.Cu") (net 3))
 (segment (start 163.825 90) (end 165.1 91.275) (width 0.2) (layer "F.Cu") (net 3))
 (segment (start 150.05 91.275) (end 150.225 91.275) (width 0.2) (layer "F.Cu") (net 3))
 (segment (start 134.1 77.375) (end 134.1 90.375) (width 0.2) (layer "F.Cu") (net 3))
 (segment (start 150.225 91.275) (end 151.5 90) (width 0.2) (layer "F.Cu") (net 3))
 (segment (start 165.1 76.475) (end 164.2 77.375) (width 0.2) (layer "F.Cu") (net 3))
 (segment (start 179.25 77.375) (end 179.25 90.375) (width 0.2) (layer "F.Cu") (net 3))
 (segment (start 178.875 90) (end 180.15 91.275) (width 0.2) (layer "F.Cu") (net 3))
 (segment (start 151.5 90) (end 163.825 90) (width 0.2) (layer "F.Cu") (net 3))
 (segment (start 148.775 90) (end 150.05 91.275) (width 0.2) (layer "F.Cu") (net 3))
 (segment (start 150.05 76.475) (end 149.15 77.375) (width 0.2) (layer "F.Cu") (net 3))
 (segment (start 149.15 90.375) (end 150.05 91.275) (width 0.2) (layer "F.Cu") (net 3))
 (segment (start 136.275 90) (end 148.775 90) (width 0.2) (layer "F.Cu") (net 3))
 (segment (start 134.1 90.375) (end 135 91.275) (width 0.2) (layer "F.Cu") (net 3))
 (segment (start 164.2 90.375) (end 165.1 91.275) (width 0.2) (layer "F.Cu") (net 3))
 (segment (start 166.375 90) (end 178.875 90) (width 0.2) (layer "F.Cu") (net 3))
 (segment (start 179.25 90.375) (end 180.15 91.275) (width 0.2) (layer "F.Cu") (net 3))
 (segment (start 164.2 77.375) (end 164.2 90.375) (width 0.2) (layer "F.Cu") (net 3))
 (segment (start 180.15 76.475) (end 179.25 77.375) (width 0.2) (layer "F.Cu") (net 3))
 (segment (start 135 76.475) (end 134.1 77.375) (width 0.2) (layer "F.Cu") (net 3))
 (segment (start 135 91.275) (end 136.275 90) (width 0.2) (layer "F.Cu") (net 3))
 (segment (start 128.75 73.090937) (end 128.75 77.25) (width 0.2) (layer "B.Cu") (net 3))
 (segment (start 132.91 68.930937) (end 128.75 73.090937) (width 0.2) (layer "B.Cu") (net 3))
 (segment (start 132.91 56.5) (end 132.91 68.930937) (width 0.2) (layer "B.Cu") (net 3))
 (segment (start 160.1 91.275) (end 161.3 92.475) (width 0.2) (layer "F.Cu") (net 1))
 (segment (start 146.525 75) (end 145.05 76.475) (width 0.2) (layer "F.Cu") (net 1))
 (segment (start 145.05 76.475) (end 143.575 75) (width 0.2) (layer "F.Cu") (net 1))
 (segment (start 145.05 91.275) (end 146.25 92.475) (width 0.2) (layer "F.Cu") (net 1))
 (segment (start 158.9 92.475) (end 160.1 91.275) (width 0.2) (layer "F.Cu") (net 1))
 (segment (start 161.3 75.275) (end 160.1 76.475) (width 0.2) (layer "F.Cu") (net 1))
 (segment (start 175.15 76.475) (end 173.95 75.275) (width 0.2) (layer "F.Cu") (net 1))
 (segment (start 130 76.475) (end 130.05 76.525) (width 0.2) (layer "F.Cu") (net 1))
 (segment (start 173.95 75.275) (end 161.3 75.275) (width 0.2) (layer "F.Cu") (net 1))
 (segment (start 131.475 75) (end 130 76.475) (width 0.2) (layer "F.Cu") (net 1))
 (segment (start 160.1 76.475) (end 158.625 75) (width 0.2) (layer "F.Cu") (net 1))
 (segment (start 143.575 75) (end 131.475 75) (width 0.2) (layer "F.Cu") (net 1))
 (segment (start 130.05 91.225) (end 130 91.275) (width 0.2) (layer "F.Cu") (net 1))
 (segment (start 131.2 92.475) (end 143.85 92.475) (width 0.2) (layer "F.Cu") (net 1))
 (segment (start 130.05 76.525) (end 130.05 91.225) (width 0.2) (layer "F.Cu") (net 1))
 (segment (start 161.3 92.475) (end 173.95 92.475) (width 0.2) (layer "F.Cu") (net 1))
 (segment (start 173.95 92.475) (end 175.15 91.275) (width 0.2) (layer "F.Cu") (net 1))
 (segment (start 130 91.275) (end 131.2 92.475) (width 0.2) (layer "F.Cu") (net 1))
 (segment (start 143.85 92.475) (end 145.05 91.275) (width 0.2) (layer "F.Cu") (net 1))
 (segment (start 146.25 92.475) (end 158.9 92.475) (width 0.2) (layer "F.Cu") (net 1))
 (segment (start 158.625 75) (end 146.525 75) (width 0.2) (layer "F.Cu") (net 1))
 (segment (start 131.3 76.972057) (end 131.3 71.106622) (width 0.2) (layer "B.Cu") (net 5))
 (segment (start 132.5 91.275) (end 132.5 78.172057) (width 0.2) (layer "B.Cu") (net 5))
 (segment (start 132.5 78.172057) (end 131.3 76.972057) (width 0.2) (layer "B.Cu") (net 5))
 (segment (start 147.55 76.475) (end 147.55 66.575686) (width 0.2) (layer "B.Cu") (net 4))
 (segment (start 147.55 91.275) (end 147.55 78.172057) (width 0.2) (layer "B.Cu") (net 2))
 (segment (start 147.55 78.172057) (end 146.35 76.972057) (width 0.2) (layer "B.Cu") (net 2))
 (segment (start 146.35 76.972057) (end 146.35 67.21) (width 0.2) (layer "B.Cu") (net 2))
 (segment (start 162.6 76.475) (end 164.5 74.575) (width 0.2) (layer "B.Cu") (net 7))
 (segment (start 164 73.377943) (end 164 63) (width 0.2) (layer "B.Cu") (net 10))
 (segment (start 161.4 75.977943) (end 164 73.377943) (width 0.2) (layer "B.Cu") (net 10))
 (segment (start 161.4 90.075) (end 161.4 75.977943) (width 0.2) (layer "B.Cu") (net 10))
 (segment (start 162.6 91.275) (end 161.4 90.075) (width 0.2) (layer "B.Cu") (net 10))
 (segment (start 177.65 76.475) (end 177.65 64.75) (width 0.2) (layer "B.Cu") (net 8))
 (segment (start 178.85 90.075) (end 178.85 65.384314) (width 0.2) (layer "B.Cu") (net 6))
 (segment (start 177.65 91.275) (end 178.85 90.075) (width 0.2) (layer "B.Cu") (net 6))
 (segment (start 163.63 56.5) (end 166.7 59.57) (width 0.2) (layer "B.Cu") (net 16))
 (segment (start 148.75 56.5) (end 163.63 56.5) (width 0.2) (layer "B.Cu") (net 16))
 (segment (start 140.83 56.5) (end 143.9 59.57) (width 0.2) (layer "B.Cu") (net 14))
 (segment (start 143.9 59.57) (end 161.62 59.57) (width 0.2) (layer "B.Cu") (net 14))
 (segment (start 146.29 58) (end 162.59 58) (width 0.2) (layer "B.Cu") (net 15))
 (segment (start 144.79 56.5) (end 146.29 58) (width 0.2) (layer "B.Cu") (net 15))
 (segment (start 162.59 58) (end 164.16 59.57) (width 0.2) (layer "B.Cu") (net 15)))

